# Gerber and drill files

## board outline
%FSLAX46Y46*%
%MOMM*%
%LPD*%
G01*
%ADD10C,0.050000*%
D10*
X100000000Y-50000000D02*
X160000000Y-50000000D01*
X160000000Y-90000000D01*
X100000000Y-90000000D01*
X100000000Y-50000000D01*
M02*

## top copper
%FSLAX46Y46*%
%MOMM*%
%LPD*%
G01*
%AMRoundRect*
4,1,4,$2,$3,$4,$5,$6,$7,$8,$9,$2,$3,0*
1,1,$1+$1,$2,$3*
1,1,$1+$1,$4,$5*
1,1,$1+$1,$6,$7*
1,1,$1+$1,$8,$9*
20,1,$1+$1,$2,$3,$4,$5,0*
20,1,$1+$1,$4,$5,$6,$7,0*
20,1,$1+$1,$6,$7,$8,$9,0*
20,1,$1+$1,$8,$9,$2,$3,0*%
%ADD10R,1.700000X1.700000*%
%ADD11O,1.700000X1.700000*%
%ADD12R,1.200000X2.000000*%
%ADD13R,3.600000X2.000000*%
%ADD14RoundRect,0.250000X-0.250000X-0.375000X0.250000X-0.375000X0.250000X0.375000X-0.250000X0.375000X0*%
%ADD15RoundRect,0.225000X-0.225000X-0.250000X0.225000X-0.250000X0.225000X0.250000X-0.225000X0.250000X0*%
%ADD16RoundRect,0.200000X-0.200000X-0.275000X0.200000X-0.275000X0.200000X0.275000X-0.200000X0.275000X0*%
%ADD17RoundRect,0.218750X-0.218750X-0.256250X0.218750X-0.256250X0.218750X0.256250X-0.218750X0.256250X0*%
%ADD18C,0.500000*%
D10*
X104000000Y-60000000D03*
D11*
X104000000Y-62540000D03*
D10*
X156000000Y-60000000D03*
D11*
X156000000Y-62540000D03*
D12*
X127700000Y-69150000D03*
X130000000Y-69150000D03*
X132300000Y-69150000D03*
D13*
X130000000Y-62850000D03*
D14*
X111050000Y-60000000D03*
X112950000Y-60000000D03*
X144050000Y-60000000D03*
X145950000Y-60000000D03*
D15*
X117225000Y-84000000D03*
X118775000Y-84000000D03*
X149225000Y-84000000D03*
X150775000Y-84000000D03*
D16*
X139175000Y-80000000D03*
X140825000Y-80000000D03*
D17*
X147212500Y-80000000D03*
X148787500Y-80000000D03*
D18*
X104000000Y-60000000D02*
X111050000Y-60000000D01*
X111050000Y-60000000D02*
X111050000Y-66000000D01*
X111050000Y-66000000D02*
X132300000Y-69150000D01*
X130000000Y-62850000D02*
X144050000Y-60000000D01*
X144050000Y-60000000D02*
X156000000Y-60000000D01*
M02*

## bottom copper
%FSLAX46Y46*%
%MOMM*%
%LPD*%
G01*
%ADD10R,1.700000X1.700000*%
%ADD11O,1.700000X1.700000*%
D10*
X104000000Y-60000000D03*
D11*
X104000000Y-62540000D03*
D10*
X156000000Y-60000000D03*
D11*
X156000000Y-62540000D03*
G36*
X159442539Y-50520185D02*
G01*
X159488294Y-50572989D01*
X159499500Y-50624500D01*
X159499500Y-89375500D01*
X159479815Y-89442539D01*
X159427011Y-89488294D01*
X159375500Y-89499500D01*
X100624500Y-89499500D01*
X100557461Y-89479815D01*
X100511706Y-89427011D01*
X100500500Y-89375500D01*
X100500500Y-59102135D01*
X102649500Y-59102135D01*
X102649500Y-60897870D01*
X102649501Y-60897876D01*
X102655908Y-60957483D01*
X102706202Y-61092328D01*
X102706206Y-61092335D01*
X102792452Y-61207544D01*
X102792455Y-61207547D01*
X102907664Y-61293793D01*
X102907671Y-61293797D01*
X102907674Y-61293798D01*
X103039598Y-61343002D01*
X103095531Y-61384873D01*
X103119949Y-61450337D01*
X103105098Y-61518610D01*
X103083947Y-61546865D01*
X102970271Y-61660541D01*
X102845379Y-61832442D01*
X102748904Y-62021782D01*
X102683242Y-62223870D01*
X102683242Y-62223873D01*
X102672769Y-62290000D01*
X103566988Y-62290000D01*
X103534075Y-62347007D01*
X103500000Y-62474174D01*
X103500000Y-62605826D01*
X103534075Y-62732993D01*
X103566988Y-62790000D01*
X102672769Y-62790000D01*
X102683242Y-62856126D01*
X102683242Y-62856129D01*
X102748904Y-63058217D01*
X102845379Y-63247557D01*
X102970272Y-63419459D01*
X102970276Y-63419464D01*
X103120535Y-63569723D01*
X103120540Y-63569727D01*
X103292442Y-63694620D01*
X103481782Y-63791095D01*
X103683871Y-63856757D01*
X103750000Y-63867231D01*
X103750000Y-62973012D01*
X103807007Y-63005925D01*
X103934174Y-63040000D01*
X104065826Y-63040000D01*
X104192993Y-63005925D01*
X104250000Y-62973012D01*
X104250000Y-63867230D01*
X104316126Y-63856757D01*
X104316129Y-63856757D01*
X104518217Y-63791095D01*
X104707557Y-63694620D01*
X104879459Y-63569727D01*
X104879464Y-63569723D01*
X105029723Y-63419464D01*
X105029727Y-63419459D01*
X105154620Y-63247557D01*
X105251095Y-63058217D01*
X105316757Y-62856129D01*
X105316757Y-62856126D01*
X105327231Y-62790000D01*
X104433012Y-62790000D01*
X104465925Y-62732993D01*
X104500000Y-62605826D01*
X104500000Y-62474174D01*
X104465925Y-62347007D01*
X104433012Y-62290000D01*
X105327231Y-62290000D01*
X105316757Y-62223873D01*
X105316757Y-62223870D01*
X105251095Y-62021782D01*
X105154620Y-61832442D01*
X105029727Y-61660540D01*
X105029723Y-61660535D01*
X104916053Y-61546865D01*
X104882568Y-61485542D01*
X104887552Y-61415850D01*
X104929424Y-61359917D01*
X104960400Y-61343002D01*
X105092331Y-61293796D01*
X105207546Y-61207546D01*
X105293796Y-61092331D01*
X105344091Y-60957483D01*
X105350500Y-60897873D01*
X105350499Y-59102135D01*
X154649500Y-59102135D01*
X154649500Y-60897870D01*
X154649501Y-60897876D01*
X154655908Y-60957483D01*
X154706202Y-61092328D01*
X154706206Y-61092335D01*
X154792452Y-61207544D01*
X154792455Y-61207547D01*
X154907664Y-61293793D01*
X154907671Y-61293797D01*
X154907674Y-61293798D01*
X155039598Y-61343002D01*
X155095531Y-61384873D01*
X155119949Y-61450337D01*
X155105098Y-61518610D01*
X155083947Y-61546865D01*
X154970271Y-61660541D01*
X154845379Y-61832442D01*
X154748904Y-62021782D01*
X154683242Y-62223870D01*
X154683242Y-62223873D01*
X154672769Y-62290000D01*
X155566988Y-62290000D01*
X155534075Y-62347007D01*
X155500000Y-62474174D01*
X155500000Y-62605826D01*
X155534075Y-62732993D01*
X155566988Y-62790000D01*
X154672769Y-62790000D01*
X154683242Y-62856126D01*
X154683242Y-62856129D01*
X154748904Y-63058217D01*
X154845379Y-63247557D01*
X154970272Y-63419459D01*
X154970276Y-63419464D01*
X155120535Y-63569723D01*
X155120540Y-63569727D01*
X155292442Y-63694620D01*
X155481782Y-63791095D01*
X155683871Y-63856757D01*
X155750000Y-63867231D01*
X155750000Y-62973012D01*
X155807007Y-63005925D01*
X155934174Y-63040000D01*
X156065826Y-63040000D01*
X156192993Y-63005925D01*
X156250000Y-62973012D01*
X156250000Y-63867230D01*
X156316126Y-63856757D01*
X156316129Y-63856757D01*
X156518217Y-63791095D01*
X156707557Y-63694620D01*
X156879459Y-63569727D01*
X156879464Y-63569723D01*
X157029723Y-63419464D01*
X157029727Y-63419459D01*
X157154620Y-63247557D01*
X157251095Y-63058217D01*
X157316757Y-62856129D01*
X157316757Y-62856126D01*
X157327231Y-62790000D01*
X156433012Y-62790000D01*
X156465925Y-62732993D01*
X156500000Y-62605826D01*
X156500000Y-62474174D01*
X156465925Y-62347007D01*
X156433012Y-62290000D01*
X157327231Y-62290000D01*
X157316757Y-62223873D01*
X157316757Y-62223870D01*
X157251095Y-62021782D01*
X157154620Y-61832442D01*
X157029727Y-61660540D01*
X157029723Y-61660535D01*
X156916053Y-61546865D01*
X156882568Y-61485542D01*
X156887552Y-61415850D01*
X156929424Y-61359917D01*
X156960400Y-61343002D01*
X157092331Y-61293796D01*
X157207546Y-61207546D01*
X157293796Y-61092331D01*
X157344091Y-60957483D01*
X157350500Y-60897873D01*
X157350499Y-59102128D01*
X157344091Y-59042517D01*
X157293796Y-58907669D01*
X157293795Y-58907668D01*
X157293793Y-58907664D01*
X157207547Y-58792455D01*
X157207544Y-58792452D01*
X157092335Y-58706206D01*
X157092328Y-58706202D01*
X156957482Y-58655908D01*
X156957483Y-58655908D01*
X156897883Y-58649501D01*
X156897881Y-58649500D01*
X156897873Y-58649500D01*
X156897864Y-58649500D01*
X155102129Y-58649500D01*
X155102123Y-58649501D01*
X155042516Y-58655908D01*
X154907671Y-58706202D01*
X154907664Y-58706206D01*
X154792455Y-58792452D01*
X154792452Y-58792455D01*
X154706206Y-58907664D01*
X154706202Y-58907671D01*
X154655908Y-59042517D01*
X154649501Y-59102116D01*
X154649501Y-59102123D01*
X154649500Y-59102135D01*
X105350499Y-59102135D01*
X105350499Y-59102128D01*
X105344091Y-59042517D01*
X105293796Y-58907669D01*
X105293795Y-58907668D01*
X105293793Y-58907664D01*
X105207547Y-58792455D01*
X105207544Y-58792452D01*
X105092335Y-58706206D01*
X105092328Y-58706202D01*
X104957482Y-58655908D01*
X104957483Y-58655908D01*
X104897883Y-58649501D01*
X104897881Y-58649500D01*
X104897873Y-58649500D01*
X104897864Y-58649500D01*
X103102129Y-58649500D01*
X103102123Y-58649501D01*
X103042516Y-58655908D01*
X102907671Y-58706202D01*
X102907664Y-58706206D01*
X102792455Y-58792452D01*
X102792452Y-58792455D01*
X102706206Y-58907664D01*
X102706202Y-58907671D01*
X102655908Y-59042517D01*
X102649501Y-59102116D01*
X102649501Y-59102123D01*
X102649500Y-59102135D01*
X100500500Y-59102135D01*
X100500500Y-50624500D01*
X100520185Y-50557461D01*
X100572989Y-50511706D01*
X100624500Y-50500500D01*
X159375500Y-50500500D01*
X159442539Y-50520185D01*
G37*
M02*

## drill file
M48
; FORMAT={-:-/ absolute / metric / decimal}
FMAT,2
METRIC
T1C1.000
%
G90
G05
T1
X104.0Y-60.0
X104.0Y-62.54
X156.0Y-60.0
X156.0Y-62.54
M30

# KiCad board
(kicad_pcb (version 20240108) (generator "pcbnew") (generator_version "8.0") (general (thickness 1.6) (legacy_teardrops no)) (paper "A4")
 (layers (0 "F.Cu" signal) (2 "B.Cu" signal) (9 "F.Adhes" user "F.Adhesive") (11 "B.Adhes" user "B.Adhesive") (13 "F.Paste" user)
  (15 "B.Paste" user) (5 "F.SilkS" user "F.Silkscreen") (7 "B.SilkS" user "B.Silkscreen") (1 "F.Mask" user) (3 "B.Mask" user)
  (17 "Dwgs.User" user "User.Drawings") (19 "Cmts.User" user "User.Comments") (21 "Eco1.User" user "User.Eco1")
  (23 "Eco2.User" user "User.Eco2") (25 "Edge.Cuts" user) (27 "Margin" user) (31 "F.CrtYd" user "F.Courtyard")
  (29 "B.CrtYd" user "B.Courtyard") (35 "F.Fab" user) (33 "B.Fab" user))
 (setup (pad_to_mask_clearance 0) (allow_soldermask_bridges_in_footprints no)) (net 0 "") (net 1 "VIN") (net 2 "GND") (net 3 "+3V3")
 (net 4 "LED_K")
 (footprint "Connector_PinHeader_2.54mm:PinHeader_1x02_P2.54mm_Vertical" (layer "F.Cu") (at 104 60)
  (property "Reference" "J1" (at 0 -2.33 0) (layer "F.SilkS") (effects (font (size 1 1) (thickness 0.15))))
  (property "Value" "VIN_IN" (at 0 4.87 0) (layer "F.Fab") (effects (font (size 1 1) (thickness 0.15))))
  (pad "1" thru_hole rect (at 0 0) (size 1.7 1.7) (drill 1) (layers "*.Cu" "*.Mask") (remove_unused_layers no) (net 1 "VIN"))
  (pad "2" thru_hole oval (at 0 2.54) (size 1.7 1.7) (drill 1) (layers "*.Cu" "*.Mask") (remove_unused_layers no) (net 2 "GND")))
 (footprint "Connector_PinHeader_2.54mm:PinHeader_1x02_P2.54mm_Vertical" (layer "F.Cu") (at 156 60)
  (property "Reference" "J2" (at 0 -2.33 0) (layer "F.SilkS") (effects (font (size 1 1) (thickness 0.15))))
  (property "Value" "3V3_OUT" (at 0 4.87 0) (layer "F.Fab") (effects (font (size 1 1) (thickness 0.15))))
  (pad "1" thru_hole rect (at 0 0) (size 1.7 1.7) (drill 1) (layers "*.Cu" "*.Mask") (remove_unused_layers no) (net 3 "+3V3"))
  (pad "2" thru_hole oval (at 0 2.54) (size 1.7 1.7) (drill 1) (layers "*.Cu" "*.Mask") (remove_unused_layers no) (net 2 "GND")))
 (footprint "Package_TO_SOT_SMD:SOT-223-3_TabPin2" (layer "F.Cu") (at 130 66)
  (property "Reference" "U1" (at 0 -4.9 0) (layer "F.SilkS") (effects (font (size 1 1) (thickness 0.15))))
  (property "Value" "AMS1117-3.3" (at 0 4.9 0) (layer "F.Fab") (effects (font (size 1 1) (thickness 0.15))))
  (pad "1" smd rect (at -2.3 3.15) (size 1.2 2) (layers "F.Cu" "F.Paste" "F.Mask") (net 2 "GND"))
  (pad "2" smd rect (at 0 3.15) (size 1.2 2) (layers "F.Cu" "F.Paste" "F.Mask") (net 3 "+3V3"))
  (pad "3" smd rect (at 2.3 3.15) (size 1.2 2) (layers "F.Cu" "F.Paste" "F.Mask") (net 1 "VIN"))
  (pad "2" smd rect (at 0 -3.15) (size 3.6 2) (layers "F.Cu" "F.Paste" "F.Mask") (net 3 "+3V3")))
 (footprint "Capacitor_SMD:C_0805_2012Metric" (layer "F.Cu") (at 112 60)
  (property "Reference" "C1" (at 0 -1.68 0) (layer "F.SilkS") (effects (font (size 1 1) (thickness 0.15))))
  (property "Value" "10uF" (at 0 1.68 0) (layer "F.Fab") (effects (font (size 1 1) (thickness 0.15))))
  (pad "1" smd roundrect (at -0.95 0) (size 1 1.25) (layers "F.Cu" "F.Paste" "F.Mask") (roundrect_rratio 0.25) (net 1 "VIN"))
  (pad "2" smd roundrect (at 0.95 0) (size 1 1.25) (layers "F.Cu" "F.Paste" "F.Mask") (roundrect_rratio 0.25) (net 2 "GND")))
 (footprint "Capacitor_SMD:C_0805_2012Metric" (layer "F.Cu") (at 145 60)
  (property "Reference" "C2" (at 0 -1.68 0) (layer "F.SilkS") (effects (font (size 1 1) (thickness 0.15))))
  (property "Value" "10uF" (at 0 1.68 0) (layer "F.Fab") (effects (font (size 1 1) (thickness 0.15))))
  (pad "1" smd roundrect (at -0.95 0) (size 1 1.25) (layers "F.Cu" "F.Paste" "F.Mask") (roundrect_rratio 0.25) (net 3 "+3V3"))
  (pad "2" smd roundrect (at 0.95 0) (size 1 1.25) (layers "F.Cu" "F.Paste" "F.Mask") (roundrect_rratio 0.25) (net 2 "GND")))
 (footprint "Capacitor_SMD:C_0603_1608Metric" (layer "F.Cu") (at 118 84)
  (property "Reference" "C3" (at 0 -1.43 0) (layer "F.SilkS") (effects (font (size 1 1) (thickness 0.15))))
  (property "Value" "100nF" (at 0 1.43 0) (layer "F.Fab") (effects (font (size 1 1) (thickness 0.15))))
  (pad "1" smd roundrect (at -0.775 0) (size 0.9 0.95) (layers "F.Cu" "F.Paste" "F.Mask") (roundrect_rratio 0.25) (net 1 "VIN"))
  (pad "2" smd roundrect (at 0.775 0) (size 0.9 0.95) (layers "F.Cu" "F.Paste" "F.Mask") (roundrect_rratio 0.25) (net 2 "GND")))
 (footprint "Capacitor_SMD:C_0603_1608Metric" (layer "F.Cu") (at 150 84)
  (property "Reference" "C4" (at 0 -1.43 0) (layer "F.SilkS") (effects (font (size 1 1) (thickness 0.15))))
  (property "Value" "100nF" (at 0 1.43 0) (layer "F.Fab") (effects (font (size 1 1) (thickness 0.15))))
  (pad "1" smd roundrect (at -0.775 0) (size 0.9 0.95) (layers "F.Cu" "F.Paste" "F.Mask") (roundrect_rratio 0.25) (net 3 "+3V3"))
  (pad "2" smd roundrect (at 0.775 0) (size 0.9 0.95) (layers "F.Cu" "F.Paste" "F.Mask") (roundrect_rratio 0.25) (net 2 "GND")))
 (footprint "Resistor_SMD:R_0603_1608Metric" (layer "F.Cu") (at 140 80)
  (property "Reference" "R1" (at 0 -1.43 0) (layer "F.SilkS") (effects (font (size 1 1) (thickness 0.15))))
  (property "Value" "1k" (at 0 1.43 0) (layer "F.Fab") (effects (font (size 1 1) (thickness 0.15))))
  (pad "1" smd roundrect (at -0.825 0) (size 0.8 0.95) (layers "F.Cu" "F.Paste" "F.Mask") (roundrect_rratio 0.25) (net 3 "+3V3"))
  (pad "2" smd roundrect (at 0.825 0) (size 0.8 0.95) (layers "F.Cu" "F.Paste" "F.Mask") (roundrect_rratio 0.25) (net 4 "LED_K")))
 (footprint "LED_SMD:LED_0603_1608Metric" (layer "F.Cu") (at 148 80)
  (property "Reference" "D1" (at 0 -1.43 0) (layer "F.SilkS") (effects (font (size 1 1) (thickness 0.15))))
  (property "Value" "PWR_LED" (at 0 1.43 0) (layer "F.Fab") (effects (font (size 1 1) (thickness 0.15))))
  (pad "1" smd roundrect (at -0.7875 0) (size 0.875 0.95) (layers "F.Cu" "F.Paste" "F.Mask") (roundrect_rratio 0.25) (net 2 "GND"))
  (pad "2" smd roundrect (at 0.7875 0) (size 0.875 0.95) (layers "F.Cu" "F.Paste" "F.Mask") (roundrect_rratio 0.25) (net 4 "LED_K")))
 (gr_rect (start 100 50) (end 160 90) (stroke (width 0.05) (type default)) (fill no) (layer "Edge.Cuts"))
 (segment (start 104 60) (end 111.05 60) (width 0.5) (layer "F.Cu") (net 1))
 (segment (start 111.05 60) (end 111.05 66) (width 0.5) (layer "F.Cu") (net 1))
 (segment (start 111.05 66) (end 132.3 69.15) (width 0.5) (layer "F.Cu") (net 1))
 (segment (start 130 62.85) (end 144.05 60) (width 0.5) (layer "F.Cu") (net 3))
 (segment (start 144.05 60) (end 156 60) (width 0.5) (layer "F.Cu") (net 3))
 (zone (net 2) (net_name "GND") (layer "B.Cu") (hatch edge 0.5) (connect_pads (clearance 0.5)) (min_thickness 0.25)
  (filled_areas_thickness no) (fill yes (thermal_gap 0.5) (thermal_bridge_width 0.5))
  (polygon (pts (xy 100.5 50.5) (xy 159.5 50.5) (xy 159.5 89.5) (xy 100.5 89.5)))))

